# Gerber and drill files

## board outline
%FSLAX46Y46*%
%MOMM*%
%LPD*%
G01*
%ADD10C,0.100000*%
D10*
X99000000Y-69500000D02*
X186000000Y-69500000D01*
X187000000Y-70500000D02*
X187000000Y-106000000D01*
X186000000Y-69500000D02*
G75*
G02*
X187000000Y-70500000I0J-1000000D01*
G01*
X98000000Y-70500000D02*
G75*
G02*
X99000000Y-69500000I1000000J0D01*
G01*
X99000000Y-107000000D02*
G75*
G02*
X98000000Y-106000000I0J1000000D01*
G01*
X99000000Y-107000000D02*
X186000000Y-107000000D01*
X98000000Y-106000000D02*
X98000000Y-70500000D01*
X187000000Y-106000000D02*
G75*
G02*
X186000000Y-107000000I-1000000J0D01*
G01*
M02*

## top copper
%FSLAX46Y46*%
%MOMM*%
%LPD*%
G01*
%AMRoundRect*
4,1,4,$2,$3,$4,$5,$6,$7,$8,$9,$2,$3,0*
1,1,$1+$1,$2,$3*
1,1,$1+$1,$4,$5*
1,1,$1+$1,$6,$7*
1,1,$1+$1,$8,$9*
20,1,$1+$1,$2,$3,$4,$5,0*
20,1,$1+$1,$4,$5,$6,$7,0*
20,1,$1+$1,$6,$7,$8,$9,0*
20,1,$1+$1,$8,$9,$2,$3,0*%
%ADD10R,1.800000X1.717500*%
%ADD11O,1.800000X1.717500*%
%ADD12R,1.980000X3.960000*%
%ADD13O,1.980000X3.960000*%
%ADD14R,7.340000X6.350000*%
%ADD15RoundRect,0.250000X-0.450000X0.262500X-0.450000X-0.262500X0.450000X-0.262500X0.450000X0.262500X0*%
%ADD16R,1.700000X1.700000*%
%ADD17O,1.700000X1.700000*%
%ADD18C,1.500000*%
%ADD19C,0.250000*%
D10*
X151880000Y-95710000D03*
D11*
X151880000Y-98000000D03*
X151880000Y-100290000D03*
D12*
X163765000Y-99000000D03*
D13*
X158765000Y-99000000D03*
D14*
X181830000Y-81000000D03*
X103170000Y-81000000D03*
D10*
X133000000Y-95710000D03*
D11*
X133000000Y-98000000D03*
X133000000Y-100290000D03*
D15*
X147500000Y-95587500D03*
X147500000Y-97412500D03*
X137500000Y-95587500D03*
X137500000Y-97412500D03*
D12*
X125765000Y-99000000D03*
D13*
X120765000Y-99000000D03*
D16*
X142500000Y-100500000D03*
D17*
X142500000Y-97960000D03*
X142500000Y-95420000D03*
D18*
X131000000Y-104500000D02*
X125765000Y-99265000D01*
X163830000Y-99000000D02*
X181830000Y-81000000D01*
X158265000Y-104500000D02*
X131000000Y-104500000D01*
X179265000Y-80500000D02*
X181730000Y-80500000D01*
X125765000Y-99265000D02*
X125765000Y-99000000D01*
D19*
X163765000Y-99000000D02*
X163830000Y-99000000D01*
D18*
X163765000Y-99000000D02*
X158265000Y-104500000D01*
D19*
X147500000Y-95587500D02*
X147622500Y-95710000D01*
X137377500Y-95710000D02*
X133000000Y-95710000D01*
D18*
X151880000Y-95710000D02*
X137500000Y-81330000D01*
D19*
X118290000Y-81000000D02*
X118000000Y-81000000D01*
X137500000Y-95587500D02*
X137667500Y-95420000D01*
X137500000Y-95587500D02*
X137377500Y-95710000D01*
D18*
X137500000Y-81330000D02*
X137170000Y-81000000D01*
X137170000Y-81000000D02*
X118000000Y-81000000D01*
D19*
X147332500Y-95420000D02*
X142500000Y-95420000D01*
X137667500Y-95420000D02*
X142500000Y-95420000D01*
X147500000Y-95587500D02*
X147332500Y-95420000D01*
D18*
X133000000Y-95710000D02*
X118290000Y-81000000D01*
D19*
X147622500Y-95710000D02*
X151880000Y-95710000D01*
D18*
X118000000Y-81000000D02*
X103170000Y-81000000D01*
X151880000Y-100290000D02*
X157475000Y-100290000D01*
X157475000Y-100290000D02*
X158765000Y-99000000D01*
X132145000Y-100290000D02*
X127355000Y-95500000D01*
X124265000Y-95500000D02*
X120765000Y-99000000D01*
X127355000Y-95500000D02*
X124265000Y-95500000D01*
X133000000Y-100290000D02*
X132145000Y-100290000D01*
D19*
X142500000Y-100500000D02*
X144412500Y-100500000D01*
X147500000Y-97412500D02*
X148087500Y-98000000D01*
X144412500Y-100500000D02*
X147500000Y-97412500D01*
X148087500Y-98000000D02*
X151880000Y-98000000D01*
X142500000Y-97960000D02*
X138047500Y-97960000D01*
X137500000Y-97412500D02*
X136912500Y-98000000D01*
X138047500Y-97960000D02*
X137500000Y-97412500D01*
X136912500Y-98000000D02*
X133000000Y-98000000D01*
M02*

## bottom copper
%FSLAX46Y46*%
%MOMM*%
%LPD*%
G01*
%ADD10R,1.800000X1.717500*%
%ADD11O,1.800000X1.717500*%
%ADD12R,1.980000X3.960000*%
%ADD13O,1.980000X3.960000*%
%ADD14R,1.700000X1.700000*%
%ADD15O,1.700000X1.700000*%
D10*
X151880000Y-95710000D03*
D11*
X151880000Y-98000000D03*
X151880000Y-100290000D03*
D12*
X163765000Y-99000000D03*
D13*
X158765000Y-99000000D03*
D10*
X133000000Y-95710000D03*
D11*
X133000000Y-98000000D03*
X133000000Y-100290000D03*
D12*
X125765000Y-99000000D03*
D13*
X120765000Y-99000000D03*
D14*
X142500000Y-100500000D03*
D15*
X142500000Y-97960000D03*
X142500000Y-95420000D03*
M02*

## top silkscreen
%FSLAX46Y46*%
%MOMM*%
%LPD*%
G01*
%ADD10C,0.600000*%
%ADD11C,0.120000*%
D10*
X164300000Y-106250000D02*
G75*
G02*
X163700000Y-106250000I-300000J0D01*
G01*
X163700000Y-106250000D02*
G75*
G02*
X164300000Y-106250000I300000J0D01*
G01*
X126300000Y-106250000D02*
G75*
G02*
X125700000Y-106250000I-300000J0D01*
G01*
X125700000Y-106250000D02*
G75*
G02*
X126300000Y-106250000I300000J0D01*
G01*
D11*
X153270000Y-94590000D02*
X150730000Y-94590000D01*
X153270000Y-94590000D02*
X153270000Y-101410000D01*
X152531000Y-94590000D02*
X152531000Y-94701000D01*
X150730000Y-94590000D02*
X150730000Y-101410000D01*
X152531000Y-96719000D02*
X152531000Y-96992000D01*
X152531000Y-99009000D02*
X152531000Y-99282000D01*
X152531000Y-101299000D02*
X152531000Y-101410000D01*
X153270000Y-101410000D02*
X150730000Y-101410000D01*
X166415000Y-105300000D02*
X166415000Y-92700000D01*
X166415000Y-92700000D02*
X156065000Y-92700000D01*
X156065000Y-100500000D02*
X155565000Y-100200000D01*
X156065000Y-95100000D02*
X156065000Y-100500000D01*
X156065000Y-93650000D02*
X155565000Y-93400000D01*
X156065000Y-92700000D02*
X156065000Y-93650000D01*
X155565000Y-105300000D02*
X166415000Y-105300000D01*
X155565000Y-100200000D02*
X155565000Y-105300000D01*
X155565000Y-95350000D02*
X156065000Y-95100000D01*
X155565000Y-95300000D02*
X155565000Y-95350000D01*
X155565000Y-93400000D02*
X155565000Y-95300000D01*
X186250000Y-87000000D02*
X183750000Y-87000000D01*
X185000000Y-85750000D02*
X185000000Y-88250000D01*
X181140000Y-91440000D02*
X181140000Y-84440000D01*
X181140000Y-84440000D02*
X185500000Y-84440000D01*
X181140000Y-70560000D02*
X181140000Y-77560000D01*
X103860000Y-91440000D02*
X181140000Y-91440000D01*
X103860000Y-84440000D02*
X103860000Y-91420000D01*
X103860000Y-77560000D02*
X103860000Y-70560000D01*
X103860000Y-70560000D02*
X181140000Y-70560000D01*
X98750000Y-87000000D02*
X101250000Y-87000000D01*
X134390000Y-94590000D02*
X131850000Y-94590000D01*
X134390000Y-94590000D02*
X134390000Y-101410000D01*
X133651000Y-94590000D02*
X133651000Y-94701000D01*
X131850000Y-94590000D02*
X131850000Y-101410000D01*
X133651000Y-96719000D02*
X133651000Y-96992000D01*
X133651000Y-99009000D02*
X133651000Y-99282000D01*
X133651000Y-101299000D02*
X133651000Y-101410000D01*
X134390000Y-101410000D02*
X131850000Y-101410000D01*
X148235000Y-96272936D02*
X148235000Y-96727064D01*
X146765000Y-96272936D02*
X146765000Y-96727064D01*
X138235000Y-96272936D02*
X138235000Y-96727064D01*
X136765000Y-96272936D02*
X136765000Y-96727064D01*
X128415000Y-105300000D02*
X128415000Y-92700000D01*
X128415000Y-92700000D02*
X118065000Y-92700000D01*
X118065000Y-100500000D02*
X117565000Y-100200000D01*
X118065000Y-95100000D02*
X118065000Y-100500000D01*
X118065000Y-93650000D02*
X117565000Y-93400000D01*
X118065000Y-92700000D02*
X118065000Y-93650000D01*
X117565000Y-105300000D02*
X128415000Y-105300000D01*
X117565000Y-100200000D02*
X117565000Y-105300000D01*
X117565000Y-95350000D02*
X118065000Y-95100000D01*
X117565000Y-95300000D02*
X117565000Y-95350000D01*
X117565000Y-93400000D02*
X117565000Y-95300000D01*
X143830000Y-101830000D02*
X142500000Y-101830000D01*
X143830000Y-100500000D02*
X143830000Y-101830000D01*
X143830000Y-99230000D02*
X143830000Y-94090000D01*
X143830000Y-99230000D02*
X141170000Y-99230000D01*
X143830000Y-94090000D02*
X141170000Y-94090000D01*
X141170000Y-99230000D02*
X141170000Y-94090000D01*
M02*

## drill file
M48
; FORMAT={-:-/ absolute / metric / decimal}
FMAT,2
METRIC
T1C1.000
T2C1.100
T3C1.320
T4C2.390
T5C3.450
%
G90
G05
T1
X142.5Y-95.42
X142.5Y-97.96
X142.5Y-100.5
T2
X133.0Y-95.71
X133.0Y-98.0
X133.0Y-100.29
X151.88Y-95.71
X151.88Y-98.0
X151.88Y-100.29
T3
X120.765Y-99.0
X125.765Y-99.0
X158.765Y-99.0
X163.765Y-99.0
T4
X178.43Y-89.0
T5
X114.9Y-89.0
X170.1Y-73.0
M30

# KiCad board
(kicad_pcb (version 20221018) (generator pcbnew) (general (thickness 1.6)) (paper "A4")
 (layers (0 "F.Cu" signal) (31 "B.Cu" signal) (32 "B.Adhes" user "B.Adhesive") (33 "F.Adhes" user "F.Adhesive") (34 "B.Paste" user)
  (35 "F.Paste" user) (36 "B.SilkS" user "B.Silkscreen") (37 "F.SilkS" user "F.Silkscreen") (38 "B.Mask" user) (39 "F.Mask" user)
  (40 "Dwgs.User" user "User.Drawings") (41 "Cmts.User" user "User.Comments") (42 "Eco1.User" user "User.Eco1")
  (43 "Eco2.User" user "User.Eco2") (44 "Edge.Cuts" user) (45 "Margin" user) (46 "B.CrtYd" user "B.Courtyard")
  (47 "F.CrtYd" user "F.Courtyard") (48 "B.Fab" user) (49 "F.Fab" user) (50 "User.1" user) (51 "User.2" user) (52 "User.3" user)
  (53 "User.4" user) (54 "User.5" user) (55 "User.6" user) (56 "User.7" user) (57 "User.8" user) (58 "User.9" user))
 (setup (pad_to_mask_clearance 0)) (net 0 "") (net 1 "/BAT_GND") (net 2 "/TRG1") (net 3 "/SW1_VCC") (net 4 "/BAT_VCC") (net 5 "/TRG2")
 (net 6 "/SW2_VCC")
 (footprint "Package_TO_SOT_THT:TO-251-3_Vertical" (layer "F.Cu") (at 151.88 95.71 -90)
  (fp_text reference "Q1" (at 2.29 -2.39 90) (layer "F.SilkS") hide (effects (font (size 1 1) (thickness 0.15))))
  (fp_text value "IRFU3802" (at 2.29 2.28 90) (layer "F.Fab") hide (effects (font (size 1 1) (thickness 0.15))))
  (fp_line (start -1.12 -1.39) (end -1.12 1.15) (stroke (width 0.12) (type solid)) (layer "F.SilkS"))
  (fp_line (start -1.12 -1.39) (end 5.7 -1.39) (stroke (width 0.12) (type solid)) (layer "F.SilkS"))
  (fp_line (start -1.12 -0.651) (end -1.009 -0.651) (stroke (width 0.12) (type solid)) (layer "F.SilkS"))
  (fp_line (start -1.12 1.15) (end 5.7 1.15) (stroke (width 0.12) (type solid)) (layer "F.SilkS"))
  (fp_line (start 1.009 -0.651) (end 1.282 -0.651) (stroke (width 0.12) (type solid)) (layer "F.SilkS"))
  (fp_line (start 3.299 -0.651) (end 3.572 -0.651) (stroke (width 0.12) (type solid)) (layer "F.SilkS"))
  (fp_line (start 5.589 -0.651) (end 5.7 -0.651) (stroke (width 0.12) (type solid)) (layer "F.SilkS"))
  (fp_line (start 5.7 -1.39) (end 5.7 1.15) (stroke (width 0.12) (type solid)) (layer "F.SilkS"))
  (pad "1" thru_hole rect (at 0 0 270) (size 1.7175 1.8) (drill 1.1) (layers "*.Cu" "*.Mask") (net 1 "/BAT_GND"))
  (pad "2" thru_hole oval (at 2.29 0 270) (size 1.7175 1.8) (drill 1.1) (layers "*.Cu" "*.Mask") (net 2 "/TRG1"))
  (pad "3" thru_hole oval (at 4.58 0 270) (size 1.7175 1.8) (drill 1.1) (layers "*.Cu" "*.Mask") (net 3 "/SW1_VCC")))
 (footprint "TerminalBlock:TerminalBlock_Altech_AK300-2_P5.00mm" (layer "F.Cu") (at 163.765 99 180)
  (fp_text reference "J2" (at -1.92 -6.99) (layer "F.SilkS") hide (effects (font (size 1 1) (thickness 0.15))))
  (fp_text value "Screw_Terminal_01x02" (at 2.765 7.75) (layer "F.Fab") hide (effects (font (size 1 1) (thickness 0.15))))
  (fp_line (start -2.65 -6.3) (end -2.65 6.3) (stroke (width 0.12) (type solid)) (layer "F.SilkS"))
  (fp_line (start -2.65 6.3) (end 7.7 6.3) (stroke (width 0.12) (type solid)) (layer "F.SilkS"))
  (fp_line (start 7.7 -1.5) (end 8.2 -1.2) (stroke (width 0.12) (type solid)) (layer "F.SilkS"))
  (fp_line (start 7.7 3.9) (end 7.7 -1.5) (stroke (width 0.12) (type solid)) (layer "F.SilkS"))
  (fp_line (start 7.7 5.35) (end 8.2 5.6) (stroke (width 0.12) (type solid)) (layer "F.SilkS"))
  (fp_line (start 7.7 6.3) (end 7.7 5.35) (stroke (width 0.12) (type solid)) (layer "F.SilkS"))
  (fp_line (start 8.2 -6.3) (end -2.65 -6.3) (stroke (width 0.12) (type solid)) (layer "F.SilkS"))
  (fp_line (start 8.2 -1.2) (end 8.2 -6.3) (stroke (width 0.12) (type solid)) (layer "F.SilkS"))
  (fp_line (start 8.2 3.65) (end 7.7 3.9) (stroke (width 0.12) (type solid)) (layer "F.SilkS"))
  (fp_line (start 8.2 3.7) (end 8.2 3.65) (stroke (width 0.12) (type solid)) (layer "F.SilkS"))
  (fp_line (start 8.2 5.6) (end 8.2 3.7) (stroke (width 0.12) (type solid)) (layer "F.SilkS"))
  (pad "1" thru_hole rect (at 0 0 180) (size 1.98 3.96) (drill 1.32) (layers "*.Cu" "*.Mask") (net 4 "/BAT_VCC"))
  (pad "2" thru_hole oval (at 5 0 180) (size 1.98 3.96) (drill 1.32) (layers "*.Cu" "*.Mask") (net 3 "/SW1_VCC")))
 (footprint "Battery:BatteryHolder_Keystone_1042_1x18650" (layer "F.Cu") (at 142.5 81 180)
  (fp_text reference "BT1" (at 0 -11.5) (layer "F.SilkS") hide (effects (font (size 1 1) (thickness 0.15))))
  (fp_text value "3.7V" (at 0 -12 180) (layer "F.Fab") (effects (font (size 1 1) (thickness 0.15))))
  (fp_line (start -43.75 -6) (end -41.25 -6) (stroke (width 0.12) (type solid)) (layer "F.SilkS"))
  (fp_line (start -42.5 -4.75) (end -42.5 -7.25) (stroke (width 0.12) (type solid)) (layer "F.SilkS"))
  (fp_line (start -38.64 -10.44) (end -38.64 -3.44) (stroke (width 0.12) (type solid)) (layer "F.SilkS"))
  (fp_line (start -38.64 -3.44) (end -43 -3.44) (stroke (width 0.12) (type solid)) (layer "F.SilkS"))
  (fp_line (start -38.64 10.44) (end -38.64 3.44) (stroke (width 0.12) (type solid)) (layer "F.SilkS"))
  (fp_line (start 38.64 -10.44) (end -38.64 -10.44) (stroke (width 0.12) (type solid)) (layer "F.SilkS"))
  (fp_line (start 38.64 -3.44) (end 38.64 -10.42) (stroke (width 0.12) (type solid)) (layer "F.SilkS"))
  (fp_line (start 38.64 3.44) (end 38.64 10.44) (stroke (width 0.12) (type solid)) (layer "F.SilkS"))
  (fp_line (start 38.64 10.44) (end -38.64 10.44) (stroke (width 0.12) (type solid)) (layer "F.SilkS"))
  (fp_line (start 43.75 -6) (end 41.25 -6) (stroke (width 0.12) (type solid)) (layer "F.SilkS"))
  (pad "" np_thru_hole circle (at -35.93 -8 180) (size 2.39 2.39) (drill 2.39) (layers "*.Cu" "*.Mask"))
  (pad "" np_thru_hole circle (at -27.6 8 180) (size 3.45 3.45) (drill 3.45) (layers "*.Cu" "*.Mask"))
  (pad "" np_thru_hole circle (at 27.6 -8 180) (size 3.45 3.45) (drill 3.45) (layers "*.Cu" "*.Mask"))
  (pad "1" smd rect (at -39.33 0 180) (size 7.34 6.35) (layers "F.Cu" "F.Paste" "F.Mask") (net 4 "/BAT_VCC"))
  (pad "2" smd rect (at 39.33 0 180) (size 7.34 6.35) (layers "F.Cu" "F.Paste" "F.Mask") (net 1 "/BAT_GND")))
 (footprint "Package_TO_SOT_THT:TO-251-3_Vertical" (layer "F.Cu") (at 133 95.71 -90)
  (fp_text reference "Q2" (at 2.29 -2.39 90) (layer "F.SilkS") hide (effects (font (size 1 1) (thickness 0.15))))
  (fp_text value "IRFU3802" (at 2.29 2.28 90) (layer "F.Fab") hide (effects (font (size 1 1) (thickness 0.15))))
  (fp_line (start -1.12 -1.39) (end -1.12 1.15) (stroke (width 0.12) (type solid)) (layer "F.SilkS"))
  (fp_line (start -1.12 -1.39) (end 5.7 -1.39) (stroke (width 0.12) (type solid)) (layer "F.SilkS"))
  (fp_line (start -1.12 -0.651) (end -1.009 -0.651) (stroke (width 0.12) (type solid)) (layer "F.SilkS"))
  (fp_line (start -1.12 1.15) (end 5.7 1.15) (stroke (width 0.12) (type solid)) (layer "F.SilkS"))
  (fp_line (start 1.009 -0.651) (end 1.282 -0.651) (stroke (width 0.12) (type solid)) (layer "F.SilkS"))
  (fp_line (start 3.299 -0.651) (end 3.572 -0.651) (stroke (width 0.12) (type solid)) (layer "F.SilkS"))
  (fp_line (start 5.589 -0.651) (end 5.7 -0.651) (stroke (width 0.12) (type solid)) (layer "F.SilkS"))
  (fp_line (start 5.7 -1.39) (end 5.7 1.15) (stroke (width 0.12) (type solid)) (layer "F.SilkS"))
  (pad "1" thru_hole rect (at 0 0 270) (size 1.7175 1.8) (drill 1.1) (layers "*.Cu" "*.Mask") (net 1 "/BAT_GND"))
  (pad "2" thru_hole oval (at 2.29 0 270) (size 1.7175 1.8) (drill 1.1) (layers "*.Cu" "*.Mask") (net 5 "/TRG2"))
  (pad "3" thru_hole oval (at 4.58 0 270) (size 1.7175 1.8) (drill 1.1) (layers "*.Cu" "*.Mask") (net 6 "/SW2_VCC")))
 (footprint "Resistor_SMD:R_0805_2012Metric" (layer "F.Cu") (at 147.5 96.5 -90)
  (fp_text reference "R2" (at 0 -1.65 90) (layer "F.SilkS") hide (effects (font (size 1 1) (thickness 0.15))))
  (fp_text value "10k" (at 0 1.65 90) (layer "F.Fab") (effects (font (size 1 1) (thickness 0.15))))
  (fp_line (start -0.227064 -0.735) (end 0.227064 -0.735) (stroke (width 0.12) (type solid)) (layer "F.SilkS"))
  (fp_line (start -0.227064 0.735) (end 0.227064 0.735) (stroke (width 0.12) (type solid)) (layer "F.SilkS"))
  (pad "1" smd roundrect (at -0.9125 0 270) (size 1.025 1.4) (layers "F.Cu" "F.Paste" "F.Mask") (roundrect_rratio 0.243902439)
   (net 1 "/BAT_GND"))
  (pad "2" smd roundrect (at 0.9125 0 270) (size 1.025 1.4) (layers "F.Cu" "F.Paste" "F.Mask") (roundrect_rratio 0.243902439)
   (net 2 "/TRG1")))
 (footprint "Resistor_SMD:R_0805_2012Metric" (layer "F.Cu") (at 137.5 96.5 -90)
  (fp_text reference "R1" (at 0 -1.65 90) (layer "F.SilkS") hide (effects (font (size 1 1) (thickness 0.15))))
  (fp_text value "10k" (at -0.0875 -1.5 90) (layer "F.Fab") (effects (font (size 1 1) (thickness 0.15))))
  (fp_line (start -0.227064 -0.735) (end 0.227064 -0.735) (stroke (width 0.12) (type solid)) (layer "F.SilkS"))
  (fp_line (start -0.227064 0.735) (end 0.227064 0.735) (stroke (width 0.12) (type solid)) (layer "F.SilkS"))
  (pad "1" smd roundrect (at -0.9125 0 270) (size 1.025 1.4) (layers "F.Cu" "F.Paste" "F.Mask") (roundrect_rratio 0.243902439)
   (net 1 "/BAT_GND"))
  (pad "2" smd roundrect (at 0.9125 0 270) (size 1.025 1.4) (layers "F.Cu" "F.Paste" "F.Mask") (roundrect_rratio 0.243902439)
   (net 5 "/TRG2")))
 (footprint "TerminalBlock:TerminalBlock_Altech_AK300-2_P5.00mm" (layer "F.Cu") (at 125.765 99 180)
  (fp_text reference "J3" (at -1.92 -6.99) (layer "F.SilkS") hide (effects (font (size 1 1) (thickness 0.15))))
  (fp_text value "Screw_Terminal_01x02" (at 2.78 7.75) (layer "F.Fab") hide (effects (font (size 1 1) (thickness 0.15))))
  (fp_line (start -2.65 -6.3) (end -2.65 6.3) (stroke (width 0.12) (type solid)) (layer "F.SilkS"))
  (fp_line (start -2.65 6.3) (end 7.7 6.3) (stroke (width 0.12) (type solid)) (layer "F.SilkS"))
  (fp_line (start 7.7 -1.5) (end 8.2 -1.2) (stroke (width 0.12) (type solid)) (layer "F.SilkS"))
  (fp_line (start 7.7 3.9) (end 7.7 -1.5) (stroke (width 0.12) (type solid)) (layer "F.SilkS"))
  (fp_line (start 7.7 5.35) (end 8.2 5.6) (stroke (width 0.12) (type solid)) (layer "F.SilkS"))
  (fp_line (start 7.7 6.3) (end 7.7 5.35) (stroke (width 0.12) (type solid)) (layer "F.SilkS"))
  (fp_line (start 8.2 -6.3) (end -2.65 -6.3) (stroke (width 0.12) (type solid)) (layer "F.SilkS"))
  (fp_line (start 8.2 -1.2) (end 8.2 -6.3) (stroke (width 0.12) (type solid)) (layer "F.SilkS"))
  (fp_line (start 8.2 3.65) (end 7.7 3.9) (stroke (width 0.12) (type solid)) (layer "F.SilkS"))
  (fp_line (start 8.2 3.7) (end 8.2 3.65) (stroke (width 0.12) (type solid)) (layer "F.SilkS"))
  (fp_line (start 8.2 5.6) (end 8.2 3.7) (stroke (width 0.12) (type solid)) (layer "F.SilkS"))
  (pad "1" thru_hole rect (at 0 0 180) (size 1.98 3.96) (drill 1.32) (layers "*.Cu" "*.Mask") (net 4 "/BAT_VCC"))
  (pad "2" thru_hole oval (at 5 0 180) (size 1.98 3.96) (drill 1.32) (layers "*.Cu" "*.Mask") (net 6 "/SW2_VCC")))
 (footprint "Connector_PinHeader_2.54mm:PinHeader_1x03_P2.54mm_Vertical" (layer "F.Cu") (at 142.5 100.5 180)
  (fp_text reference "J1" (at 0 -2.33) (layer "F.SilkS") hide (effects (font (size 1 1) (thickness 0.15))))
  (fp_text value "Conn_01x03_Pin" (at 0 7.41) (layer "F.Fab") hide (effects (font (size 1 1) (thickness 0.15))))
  (fp_line (start -1.33 -1.33) (end 0 -1.33) (stroke (width 0.12) (type solid)) (layer "F.SilkS"))
  (fp_line (start -1.33 0) (end -1.33 -1.33) (stroke (width 0.12) (type solid)) (layer "F.SilkS"))
  (fp_line (start -1.33 1.27) (end -1.33 6.41) (stroke (width 0.12) (type solid)) (layer "F.SilkS"))
  (fp_line (start -1.33 1.27) (end 1.33 1.27) (stroke (width 0.12) (type solid)) (layer "F.SilkS"))
  (fp_line (start -1.33 6.41) (end 1.33 6.41) (stroke (width 0.12) (type solid)) (layer "F.SilkS"))
  (fp_line (start 1.33 1.27) (end 1.33 6.41) (stroke (width 0.12) (type solid)) (layer "F.SilkS"))
  (pad "1" thru_hole rect (at 0 0 180) (size 1.7 1.7) (drill 1) (layers "*.Cu" "*.Mask") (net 2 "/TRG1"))
  (pad "2" thru_hole oval (at 0 2.54 180) (size 1.7 1.7) (drill 1) (layers "*.Cu" "*.Mask") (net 5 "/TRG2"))
  (pad "3" thru_hole oval (at 0 5.08 180) (size 1.7 1.7) (drill 1) (layers "*.Cu" "*.Mask") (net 1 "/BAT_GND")))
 (gr_circle (center 164 106.25) (end 164.5 106.25) (stroke (width 0.2) (type solid)) (fill solid) (layer "F.SilkS"))
 (gr_circle (center 126 106.25) (end 126.5 106.25) (stroke (width 0.2) (type solid)) (fill solid) (layer "F.SilkS"))
 (gr_line (start 99 69.5) (end 186 69.5) (stroke (width 0.1) (type default)) (layer "Edge.Cuts"))
 (gr_line (start 187 70.5) (end 187 106) (stroke (width 0.1) (type default)) (layer "Edge.Cuts"))
 (gr_arc (start 186 69.5) (mid 186.707107 69.792893) (end 187 70.5) (stroke (width 0.1) (type default)) (layer "Edge.Cuts"))
 (gr_arc (start 98 70.5) (mid 98.292893 69.792893) (end 99 69.5) (stroke (width 0.1) (type default)) (layer "Edge.Cuts"))
 (gr_arc (start 99 107) (mid 98.292893 106.707107) (end 98 106) (stroke (width 0.1) (type default)) (layer "Edge.Cuts"))
 (gr_line (start 99 107) (end 186 107) (stroke (width 0.1) (type default)) (layer "Edge.Cuts"))
 (gr_line (start 98 106) (end 98 70.5) (stroke (width 0.1) (type default)) (layer "Edge.Cuts"))
 (gr_arc (start 187 106) (mid 186.707107 106.707107) (end 186 107) (stroke (width 0.1) (type default)) (layer "Edge.Cuts"))
 (segment (start 131 104.5) (end 125.765 99.265) (width 1.5) (layer "F.Cu") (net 4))
 (segment (start 163.83 99) (end 181.83 81) (width 1.5) (layer "F.Cu") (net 4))
 (segment (start 158.265 104.5) (end 131 104.5) (width 1.5) (layer "F.Cu") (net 4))
 (segment (start 179.265 80.5) (end 181.73 80.5) (width 1.5) (layer "F.Cu") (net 4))
 (segment (start 125.765 99.265) (end 125.765 99) (width 1.5) (layer "F.Cu") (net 4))
 (segment (start 163.765 99) (end 163.83 99) (width 0.25) (layer "F.Cu") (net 4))
 (segment (start 163.765 99) (end 158.265 104.5) (width 1.5) (layer "F.Cu") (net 4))
 (segment (start 147.5 95.5875) (end 147.6225 95.71) (width 0.25) (layer "F.Cu") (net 1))
 (segment (start 137.3775 95.71) (end 133 95.71) (width 0.25) (layer "F.Cu") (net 1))
 (segment (start 151.88 95.71) (end 137.5 81.33) (width 1.5) (layer "F.Cu") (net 1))
 (segment (start 118.29 81) (end 118 81) (width 0.25) (layer "F.Cu") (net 1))
 (segment (start 137.5 95.5875) (end 137.6675 95.42) (width 0.25) (layer "F.Cu") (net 1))
 (segment (start 137.5 95.5875) (end 137.3775 95.71) (width 0.25) (layer "F.Cu") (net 1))
 (segment (start 137.5 81.33) (end 137.17 81) (width 1.5) (layer "F.Cu") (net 1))
 (segment (start 137.17 81) (end 118 81) (width 1.5) (layer "F.Cu") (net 1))
 (segment (start 147.3325 95.42) (end 142.5 95.42) (width 0.25) (layer "F.Cu") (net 1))
 (segment (start 137.6675 95.42) (end 142.5 95.42) (width 0.25) (layer "F.Cu") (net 1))
 (segment (start 147.5 95.5875) (end 147.3325 95.42) (width 0.25) (layer "F.Cu") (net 1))
 (segment (start 133 95.71) (end 118.29 81) (width 1.5) (layer "F.Cu") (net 1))
 (segment (start 147.6225 95.71) (end 151.88 95.71) (width 0.25) (layer "F.Cu") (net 1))
 (segment (start 118 81) (end 103.17 81) (width 1.5) (layer "F.Cu") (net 1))
 (segment (start 151.88 100.29) (end 157.475 100.29) (width 1.5) (layer "F.Cu") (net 3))
 (segment (start 157.475 100.29) (end 158.765 99) (width 1.5) (layer "F.Cu") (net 3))
 (segment (start 132.145 100.29) (end 127.355 95.5) (width 1.5) (layer "F.Cu") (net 6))
 (segment (start 124.265 95.5) (end 120.765 99) (width 1.5) (layer "F.Cu") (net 6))
 (segment (start 127.355 95.5) (end 124.265 95.5) (width 1.5) (layer "F.Cu") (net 6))
 (segment (start 133 100.29) (end 132.145 100.29) (width 1.5) (layer "F.Cu") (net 6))
 (segment (start 142.5 100.5) (end 144.4125 100.5) (width 0.25) (layer "F.Cu") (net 2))
 (segment (start 147.5 97.4125) (end 148.0875 98) (width 0.25) (layer "F.Cu") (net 2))
 (segment (start 144.4125 100.5) (end 147.5 97.4125) (width 0.25) (layer "F.Cu") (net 2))
 (segment (start 148.0875 98) (end 151.88 98) (width 0.25) (layer "F.Cu") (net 2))
 (segment (start 142.5 97.96) (end 138.0475 97.96) (width 0.25) (layer "F.Cu") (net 5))
 (segment (start 137.5 97.4125) (end 136.9125 98) (width 0.25) (layer "F.Cu") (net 5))
 (segment (start 138.0475 97.96) (end 137.5 97.4125) (width 0.25) (layer "F.Cu") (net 5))
 (segment (start 136.9125 98) (end 133 98) (width 0.25) (layer "F.Cu") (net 5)))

